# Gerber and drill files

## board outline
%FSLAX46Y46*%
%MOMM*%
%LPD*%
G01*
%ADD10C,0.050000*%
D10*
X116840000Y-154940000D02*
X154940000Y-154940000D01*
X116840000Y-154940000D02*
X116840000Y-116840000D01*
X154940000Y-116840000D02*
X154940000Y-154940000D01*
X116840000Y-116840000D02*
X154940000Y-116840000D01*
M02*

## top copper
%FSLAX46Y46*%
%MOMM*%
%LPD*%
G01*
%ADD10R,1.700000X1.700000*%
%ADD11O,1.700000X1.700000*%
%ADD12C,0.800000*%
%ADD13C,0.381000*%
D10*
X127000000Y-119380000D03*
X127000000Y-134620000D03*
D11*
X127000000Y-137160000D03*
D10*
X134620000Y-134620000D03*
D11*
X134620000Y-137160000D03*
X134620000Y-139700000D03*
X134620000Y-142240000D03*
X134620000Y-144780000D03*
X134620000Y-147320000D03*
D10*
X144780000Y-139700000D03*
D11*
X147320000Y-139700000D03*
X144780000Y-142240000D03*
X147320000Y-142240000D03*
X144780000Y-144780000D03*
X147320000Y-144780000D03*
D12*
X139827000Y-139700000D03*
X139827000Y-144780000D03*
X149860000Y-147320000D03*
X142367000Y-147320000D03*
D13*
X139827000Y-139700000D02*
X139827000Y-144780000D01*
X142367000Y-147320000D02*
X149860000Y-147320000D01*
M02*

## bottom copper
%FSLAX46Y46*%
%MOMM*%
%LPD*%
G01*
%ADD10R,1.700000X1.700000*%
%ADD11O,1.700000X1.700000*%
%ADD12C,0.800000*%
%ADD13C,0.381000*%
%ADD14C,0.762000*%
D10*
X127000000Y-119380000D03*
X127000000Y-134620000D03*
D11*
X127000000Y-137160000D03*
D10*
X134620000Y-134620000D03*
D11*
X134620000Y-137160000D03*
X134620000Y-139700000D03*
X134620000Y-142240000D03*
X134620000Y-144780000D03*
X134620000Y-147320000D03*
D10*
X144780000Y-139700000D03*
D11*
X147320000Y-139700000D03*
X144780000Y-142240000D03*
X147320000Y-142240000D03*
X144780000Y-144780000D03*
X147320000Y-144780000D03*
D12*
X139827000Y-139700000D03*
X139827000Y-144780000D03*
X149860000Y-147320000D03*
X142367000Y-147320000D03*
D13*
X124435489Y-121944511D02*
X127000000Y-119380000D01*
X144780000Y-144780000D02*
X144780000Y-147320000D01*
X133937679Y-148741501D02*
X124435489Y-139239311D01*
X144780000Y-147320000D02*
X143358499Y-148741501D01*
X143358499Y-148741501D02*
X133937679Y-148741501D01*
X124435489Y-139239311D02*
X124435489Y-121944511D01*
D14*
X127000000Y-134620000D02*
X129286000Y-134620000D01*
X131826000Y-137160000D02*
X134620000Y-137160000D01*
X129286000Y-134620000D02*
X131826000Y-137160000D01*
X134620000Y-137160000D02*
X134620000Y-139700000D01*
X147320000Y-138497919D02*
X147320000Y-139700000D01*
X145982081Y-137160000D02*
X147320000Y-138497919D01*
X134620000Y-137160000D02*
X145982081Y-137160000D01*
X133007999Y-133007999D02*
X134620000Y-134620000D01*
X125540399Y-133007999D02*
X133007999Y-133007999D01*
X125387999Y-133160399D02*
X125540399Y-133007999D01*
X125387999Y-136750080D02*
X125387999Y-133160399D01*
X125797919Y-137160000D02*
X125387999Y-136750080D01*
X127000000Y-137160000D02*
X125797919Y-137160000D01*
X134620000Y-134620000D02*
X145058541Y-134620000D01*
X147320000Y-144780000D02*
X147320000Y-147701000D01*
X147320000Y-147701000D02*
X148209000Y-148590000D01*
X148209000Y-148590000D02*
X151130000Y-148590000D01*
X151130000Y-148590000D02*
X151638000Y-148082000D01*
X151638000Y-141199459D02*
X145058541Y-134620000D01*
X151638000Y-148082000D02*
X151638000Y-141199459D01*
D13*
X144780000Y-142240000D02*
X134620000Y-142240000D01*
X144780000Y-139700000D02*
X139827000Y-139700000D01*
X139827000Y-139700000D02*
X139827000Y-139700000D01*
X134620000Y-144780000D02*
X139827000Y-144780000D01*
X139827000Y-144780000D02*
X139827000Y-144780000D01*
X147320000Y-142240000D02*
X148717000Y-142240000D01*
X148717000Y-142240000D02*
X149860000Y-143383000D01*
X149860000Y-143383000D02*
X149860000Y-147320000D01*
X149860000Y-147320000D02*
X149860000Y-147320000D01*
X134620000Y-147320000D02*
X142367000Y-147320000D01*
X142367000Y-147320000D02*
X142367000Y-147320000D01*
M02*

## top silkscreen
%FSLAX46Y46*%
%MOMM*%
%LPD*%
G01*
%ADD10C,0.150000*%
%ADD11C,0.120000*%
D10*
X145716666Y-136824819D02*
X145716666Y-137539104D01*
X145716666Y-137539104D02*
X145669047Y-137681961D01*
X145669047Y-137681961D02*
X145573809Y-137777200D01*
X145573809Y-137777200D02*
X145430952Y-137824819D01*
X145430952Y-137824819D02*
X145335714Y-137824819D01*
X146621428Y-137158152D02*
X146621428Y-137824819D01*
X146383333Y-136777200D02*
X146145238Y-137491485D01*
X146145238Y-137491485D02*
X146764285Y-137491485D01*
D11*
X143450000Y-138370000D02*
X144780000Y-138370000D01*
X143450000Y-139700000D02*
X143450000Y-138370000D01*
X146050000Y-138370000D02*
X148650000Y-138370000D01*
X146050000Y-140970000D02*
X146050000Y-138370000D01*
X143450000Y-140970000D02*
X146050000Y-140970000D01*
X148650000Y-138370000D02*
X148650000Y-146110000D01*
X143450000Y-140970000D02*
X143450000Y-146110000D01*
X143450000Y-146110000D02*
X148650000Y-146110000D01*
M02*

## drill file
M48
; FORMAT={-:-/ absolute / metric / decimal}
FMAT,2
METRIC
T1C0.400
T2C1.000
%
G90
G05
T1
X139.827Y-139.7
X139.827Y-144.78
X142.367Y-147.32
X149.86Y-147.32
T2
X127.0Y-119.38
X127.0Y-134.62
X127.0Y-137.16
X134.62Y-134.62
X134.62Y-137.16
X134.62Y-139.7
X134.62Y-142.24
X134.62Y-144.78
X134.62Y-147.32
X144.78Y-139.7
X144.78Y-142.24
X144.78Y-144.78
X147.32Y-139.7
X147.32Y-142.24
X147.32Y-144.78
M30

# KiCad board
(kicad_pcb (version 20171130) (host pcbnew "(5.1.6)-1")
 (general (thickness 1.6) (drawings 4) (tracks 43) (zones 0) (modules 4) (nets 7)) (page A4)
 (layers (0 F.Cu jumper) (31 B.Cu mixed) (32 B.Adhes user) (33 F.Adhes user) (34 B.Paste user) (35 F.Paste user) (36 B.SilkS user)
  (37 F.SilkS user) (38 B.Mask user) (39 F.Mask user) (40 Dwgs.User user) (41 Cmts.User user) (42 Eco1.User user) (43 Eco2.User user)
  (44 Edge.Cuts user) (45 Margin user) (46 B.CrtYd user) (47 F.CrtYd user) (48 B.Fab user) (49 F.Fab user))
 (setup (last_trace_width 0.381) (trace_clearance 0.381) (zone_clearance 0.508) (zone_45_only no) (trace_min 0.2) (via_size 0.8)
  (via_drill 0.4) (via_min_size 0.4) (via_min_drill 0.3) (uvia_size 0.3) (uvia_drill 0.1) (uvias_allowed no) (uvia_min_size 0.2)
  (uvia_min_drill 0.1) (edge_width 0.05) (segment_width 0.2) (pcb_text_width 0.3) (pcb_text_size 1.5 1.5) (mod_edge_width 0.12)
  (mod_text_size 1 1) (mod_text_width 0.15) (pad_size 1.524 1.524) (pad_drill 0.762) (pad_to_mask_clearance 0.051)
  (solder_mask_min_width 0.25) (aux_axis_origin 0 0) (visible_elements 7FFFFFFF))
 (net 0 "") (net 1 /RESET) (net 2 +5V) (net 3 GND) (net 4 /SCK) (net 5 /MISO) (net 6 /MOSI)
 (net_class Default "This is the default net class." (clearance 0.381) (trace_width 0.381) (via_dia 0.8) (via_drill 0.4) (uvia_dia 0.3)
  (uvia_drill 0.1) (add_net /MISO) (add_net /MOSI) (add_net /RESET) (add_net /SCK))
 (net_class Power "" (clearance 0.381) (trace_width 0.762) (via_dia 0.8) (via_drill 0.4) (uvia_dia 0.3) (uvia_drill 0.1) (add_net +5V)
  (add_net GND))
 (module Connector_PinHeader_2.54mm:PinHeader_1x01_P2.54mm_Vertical (layer B.Cu) (at 127 119.38)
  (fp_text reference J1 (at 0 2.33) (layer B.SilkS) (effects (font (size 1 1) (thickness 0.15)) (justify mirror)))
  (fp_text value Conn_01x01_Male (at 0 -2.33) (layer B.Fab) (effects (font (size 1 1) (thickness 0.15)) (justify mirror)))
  (pad 1 thru_hole rect (at 0 0) (size 1.7 1.7) (drill 1) (layers *.Cu *.Mask) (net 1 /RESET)))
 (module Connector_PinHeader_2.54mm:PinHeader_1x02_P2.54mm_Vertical (layer B.Cu) (at 127 134.62 180)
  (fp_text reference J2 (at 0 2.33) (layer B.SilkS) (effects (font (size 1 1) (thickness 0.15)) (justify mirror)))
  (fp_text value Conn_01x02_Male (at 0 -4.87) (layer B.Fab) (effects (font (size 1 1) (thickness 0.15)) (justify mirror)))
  (pad 1 thru_hole rect (at 0 0 180) (size 1.7 1.7) (drill 1) (layers *.Cu *.Mask) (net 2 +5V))
  (pad 2 thru_hole oval (at 0 -2.54 180) (size 1.7 1.7) (drill 1) (layers *.Cu *.Mask) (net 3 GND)))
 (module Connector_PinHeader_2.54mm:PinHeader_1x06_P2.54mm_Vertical (layer B.Cu) (at 134.62 134.62 180)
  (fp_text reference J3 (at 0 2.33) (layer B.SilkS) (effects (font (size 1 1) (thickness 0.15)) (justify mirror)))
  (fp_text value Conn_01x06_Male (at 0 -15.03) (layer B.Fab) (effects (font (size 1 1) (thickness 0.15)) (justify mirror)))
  (pad 1 thru_hole rect (at 0 0 180) (size 1.7 1.7) (drill 1) (layers *.Cu *.Mask) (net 3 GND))
  (pad 2 thru_hole oval (at 0 -2.54 180) (size 1.7 1.7) (drill 1) (layers *.Cu *.Mask) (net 2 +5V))
  (pad 3 thru_hole oval (at 0 -5.08 180) (size 1.7 1.7) (drill 1) (layers *.Cu *.Mask) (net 2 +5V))
  (pad 4 thru_hole oval (at 0 -7.62 180) (size 1.7 1.7) (drill 1) (layers *.Cu *.Mask) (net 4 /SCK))
  (pad 5 thru_hole oval (at 0 -10.16 180) (size 1.7 1.7) (drill 1) (layers *.Cu *.Mask) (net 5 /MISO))
  (pad 6 thru_hole oval (at 0 -12.7 180) (size 1.7 1.7) (drill 1) (layers *.Cu *.Mask) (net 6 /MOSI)))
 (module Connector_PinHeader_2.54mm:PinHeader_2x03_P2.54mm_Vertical (layer F.Cu) (at 144.78 139.7)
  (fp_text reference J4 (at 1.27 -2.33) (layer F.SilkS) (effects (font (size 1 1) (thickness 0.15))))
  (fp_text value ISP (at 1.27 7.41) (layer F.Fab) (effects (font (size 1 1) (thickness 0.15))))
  (fp_line (start -1.33 -1.33) (end 0 -1.33) (layer F.SilkS) (width 0.12))
  (fp_line (start -1.33 0) (end -1.33 -1.33) (layer F.SilkS) (width 0.12))
  (fp_line (start 1.27 -1.33) (end 3.87 -1.33) (layer F.SilkS) (width 0.12))
  (fp_line (start 1.27 1.27) (end 1.27 -1.33) (layer F.SilkS) (width 0.12))
  (fp_line (start -1.33 1.27) (end 1.27 1.27) (layer F.SilkS) (width 0.12))
  (fp_line (start 3.87 -1.33) (end 3.87 6.41) (layer F.SilkS) (width 0.12))
  (fp_line (start -1.33 1.27) (end -1.33 6.41) (layer F.SilkS) (width 0.12))
  (fp_line (start -1.33 6.41) (end 3.87 6.41) (layer F.SilkS) (width 0.12))
  (pad 1 thru_hole rect (at 0 0) (size 1.7 1.7) (drill 1) (layers *.Cu *.Mask) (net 5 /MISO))
  (pad 2 thru_hole oval (at 2.54 0) (size 1.7 1.7) (drill 1) (layers *.Cu *.Mask) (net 2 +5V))
  (pad 3 thru_hole oval (at 0 2.54) (size 1.7 1.7) (drill 1) (layers *.Cu *.Mask) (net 4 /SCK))
  (pad 4 thru_hole oval (at 2.54 2.54) (size 1.7 1.7) (drill 1) (layers *.Cu *.Mask) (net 6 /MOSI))
  (pad 5 thru_hole oval (at 0 5.08) (size 1.7 1.7) (drill 1) (layers *.Cu *.Mask) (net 1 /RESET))
  (pad 6 thru_hole oval (at 2.54 5.08) (size 1.7 1.7) (drill 1) (layers *.Cu *.Mask) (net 3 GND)))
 (gr_line (start 116.84 154.94) (end 154.94 154.94) (layer Edge.Cuts) (width 0.05))
 (gr_line (start 116.84 154.94) (end 116.84 116.84) (layer Edge.Cuts) (width 0.05))
 (gr_line (start 154.94 116.84) (end 154.94 154.94) (layer Edge.Cuts) (width 0.05))
 (gr_line (start 116.84 116.84) (end 154.94 116.84) (layer Edge.Cuts) (width 0.05))
 (segment (start 124.435489 121.944511) (end 127 119.38) (width 0.381) (layer B.Cu) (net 1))
 (segment (start 144.78 144.78) (end 144.78 147.32) (width 0.381) (layer B.Cu) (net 1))
 (segment (start 133.937679 148.741501) (end 124.435489 139.239311) (width 0.381) (layer B.Cu) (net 1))
 (segment (start 144.78 147.32) (end 143.358499 148.741501) (width 0.381) (layer B.Cu) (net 1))
 (segment (start 143.358499 148.741501) (end 133.937679 148.741501) (width 0.381) (layer B.Cu) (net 1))
 (segment (start 124.435489 139.239311) (end 124.435489 121.944511) (width 0.381) (layer B.Cu) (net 1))
 (segment (start 127 134.62) (end 129.286 134.62) (width 0.762) (layer B.Cu) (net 2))
 (segment (start 131.826 137.16) (end 134.62 137.16) (width 0.762) (layer B.Cu) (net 2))
 (segment (start 129.286 134.62) (end 131.826 137.16) (width 0.762) (layer B.Cu) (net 2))
 (segment (start 134.62 137.16) (end 134.62 139.7) (width 0.762) (layer B.Cu) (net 2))
 (segment (start 147.32 138.497919) (end 147.32 139.7) (width 0.762) (layer B.Cu) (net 2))
 (segment (start 145.982081 137.16) (end 147.32 138.497919) (width 0.762) (layer B.Cu) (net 2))
 (segment (start 134.62 137.16) (end 145.982081 137.16) (width 0.762) (layer B.Cu) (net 2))
 (segment (start 133.007999 133.007999) (end 134.62 134.62) (width 0.762) (layer B.Cu) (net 3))
 (segment (start 125.540399 133.007999) (end 133.007999 133.007999) (width 0.762) (layer B.Cu) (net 3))
 (segment (start 125.387999 133.160399) (end 125.540399 133.007999) (width 0.762) (layer B.Cu) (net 3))
 (segment (start 125.387999 136.75008) (end 125.387999 133.160399) (width 0.762) (layer B.Cu) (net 3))
 (segment (start 125.797919 137.16) (end 125.387999 136.75008) (width 0.762) (layer B.Cu) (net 3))
 (segment (start 127 137.16) (end 125.797919 137.16) (width 0.762) (layer B.Cu) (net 3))
 (segment (start 134.62 134.62) (end 145.058541 134.62) (width 0.762) (layer B.Cu) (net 3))
 (segment (start 147.32 144.78) (end 147.32 147.701) (width 0.762) (layer B.Cu) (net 3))
 (segment (start 147.32 147.701) (end 148.209 148.59) (width 0.762) (layer B.Cu) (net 3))
 (segment (start 148.209 148.59) (end 151.13 148.59) (width 0.762) (layer B.Cu) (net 3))
 (segment (start 151.13 148.59) (end 151.638 148.082) (width 0.762) (layer B.Cu) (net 3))
 (segment (start 151.638 141.199459) (end 145.058541 134.62) (width 0.762) (layer B.Cu) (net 3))
 (segment (start 151.638 148.082) (end 151.638 141.199459) (width 0.762) (layer B.Cu) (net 3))
 (segment (start 144.78 142.24) (end 134.62 142.24) (width 0.381) (layer B.Cu) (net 4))
 (segment (start 144.78 139.7) (end 139.827 139.7) (width 0.381) (layer B.Cu) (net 5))
 (segment (start 139.827 139.7) (end 139.827 139.7) (width 0.381) (layer B.Cu) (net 5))
 (via (at 139.827 139.7) (size 0.8) (drill 0.4) (layers F.Cu B.Cu) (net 5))
 (segment (start 134.62 144.78) (end 139.827 144.78) (width 0.381) (layer B.Cu) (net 5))
 (segment (start 139.827 144.78) (end 139.827 144.78) (width 0.381) (layer B.Cu) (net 5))
 (via (at 139.827 144.78) (size 0.8) (drill 0.4) (layers F.Cu B.Cu) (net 5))
 (segment (start 139.827 139.7) (end 139.827 144.78) (width 0.381) (layer F.Cu) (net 5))
 (segment (start 147.32 142.24) (end 148.717 142.24) (width 0.381) (layer B.Cu) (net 6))
 (segment (start 148.717 142.24) (end 149.86 143.383) (width 0.381) (layer B.Cu) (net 6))
 (segment (start 149.86 143.383) (end 149.86 147.32) (width 0.381) (layer B.Cu) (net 6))
 (segment (start 149.86 147.32) (end 149.86 147.32) (width 0.381) (layer B.Cu) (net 6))
 (via (at 149.86 147.32) (size 0.8) (drill 0.4) (layers F.Cu B.Cu) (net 6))
 (segment (start 134.62 147.32) (end 142.367 147.32) (width 0.381) (layer B.Cu) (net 6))
 (segment (start 142.367 147.32) (end 142.367 147.32) (width 0.381) (layer B.Cu) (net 6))
 (via (at 142.367 147.32) (size 0.8) (drill 0.4) (layers F.Cu B.Cu) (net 6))
 (segment (start 142.367 147.32) (end 149.86 147.32) (width 0.381) (layer F.Cu) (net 6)))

